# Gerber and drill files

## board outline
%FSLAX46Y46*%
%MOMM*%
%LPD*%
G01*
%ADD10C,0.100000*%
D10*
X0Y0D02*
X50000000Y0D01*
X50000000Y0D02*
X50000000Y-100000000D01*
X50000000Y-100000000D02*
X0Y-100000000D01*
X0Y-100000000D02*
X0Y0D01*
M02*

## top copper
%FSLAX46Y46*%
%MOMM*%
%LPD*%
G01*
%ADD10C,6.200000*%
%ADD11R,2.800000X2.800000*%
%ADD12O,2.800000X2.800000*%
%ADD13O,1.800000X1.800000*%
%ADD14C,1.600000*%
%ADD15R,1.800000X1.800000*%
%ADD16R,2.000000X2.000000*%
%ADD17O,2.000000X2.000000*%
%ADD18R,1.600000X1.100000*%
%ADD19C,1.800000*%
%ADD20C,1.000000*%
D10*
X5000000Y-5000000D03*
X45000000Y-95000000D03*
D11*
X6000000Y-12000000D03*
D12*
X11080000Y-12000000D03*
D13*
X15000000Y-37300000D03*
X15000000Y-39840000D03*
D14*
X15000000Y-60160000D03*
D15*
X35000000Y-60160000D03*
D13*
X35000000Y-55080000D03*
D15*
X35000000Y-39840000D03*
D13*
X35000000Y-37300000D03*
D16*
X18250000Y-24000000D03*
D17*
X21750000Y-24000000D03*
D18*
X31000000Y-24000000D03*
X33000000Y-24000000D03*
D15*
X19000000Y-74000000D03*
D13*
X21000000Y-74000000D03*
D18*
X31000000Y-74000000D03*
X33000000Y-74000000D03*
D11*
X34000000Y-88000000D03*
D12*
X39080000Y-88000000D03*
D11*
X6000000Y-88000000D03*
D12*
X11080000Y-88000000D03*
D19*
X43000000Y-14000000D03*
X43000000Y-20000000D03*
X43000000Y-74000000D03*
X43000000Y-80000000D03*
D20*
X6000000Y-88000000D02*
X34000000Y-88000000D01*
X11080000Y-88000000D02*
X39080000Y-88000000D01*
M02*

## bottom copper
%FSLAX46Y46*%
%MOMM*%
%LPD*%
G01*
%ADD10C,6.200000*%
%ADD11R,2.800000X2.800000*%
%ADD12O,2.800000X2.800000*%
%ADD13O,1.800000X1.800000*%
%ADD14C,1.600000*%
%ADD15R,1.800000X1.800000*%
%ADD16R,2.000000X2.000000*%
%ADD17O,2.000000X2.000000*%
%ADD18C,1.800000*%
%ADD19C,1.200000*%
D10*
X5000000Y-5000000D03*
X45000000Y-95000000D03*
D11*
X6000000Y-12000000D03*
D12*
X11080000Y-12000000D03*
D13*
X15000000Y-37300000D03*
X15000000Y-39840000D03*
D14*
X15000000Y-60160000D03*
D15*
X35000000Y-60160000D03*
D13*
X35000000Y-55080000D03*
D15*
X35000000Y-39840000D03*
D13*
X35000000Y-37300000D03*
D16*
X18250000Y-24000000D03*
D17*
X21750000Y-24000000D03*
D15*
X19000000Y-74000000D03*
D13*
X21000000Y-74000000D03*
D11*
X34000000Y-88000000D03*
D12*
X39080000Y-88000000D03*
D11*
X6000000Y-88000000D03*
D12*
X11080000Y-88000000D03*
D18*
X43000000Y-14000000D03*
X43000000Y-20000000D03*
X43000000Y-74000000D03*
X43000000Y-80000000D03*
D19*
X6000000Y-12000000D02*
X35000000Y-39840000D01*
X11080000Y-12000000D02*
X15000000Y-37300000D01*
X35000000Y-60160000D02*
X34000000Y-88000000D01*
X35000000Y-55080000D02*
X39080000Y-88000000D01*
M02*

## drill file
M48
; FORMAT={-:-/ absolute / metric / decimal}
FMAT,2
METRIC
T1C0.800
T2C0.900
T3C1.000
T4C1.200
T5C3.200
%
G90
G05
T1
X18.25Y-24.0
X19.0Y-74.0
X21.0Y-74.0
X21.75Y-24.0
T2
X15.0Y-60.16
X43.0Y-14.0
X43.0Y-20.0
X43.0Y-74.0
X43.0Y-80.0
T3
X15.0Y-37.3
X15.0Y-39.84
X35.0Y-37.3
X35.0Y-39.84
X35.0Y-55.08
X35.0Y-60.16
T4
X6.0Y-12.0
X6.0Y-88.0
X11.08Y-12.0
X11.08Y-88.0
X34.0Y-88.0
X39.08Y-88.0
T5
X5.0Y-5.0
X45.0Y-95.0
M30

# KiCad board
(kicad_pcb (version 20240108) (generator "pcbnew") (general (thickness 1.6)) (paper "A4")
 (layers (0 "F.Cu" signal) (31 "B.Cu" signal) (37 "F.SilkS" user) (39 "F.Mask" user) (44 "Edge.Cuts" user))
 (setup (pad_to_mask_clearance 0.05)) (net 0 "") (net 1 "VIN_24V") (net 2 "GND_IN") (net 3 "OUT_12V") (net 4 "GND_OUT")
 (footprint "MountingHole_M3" (layer "F.Cu") (at 5 5)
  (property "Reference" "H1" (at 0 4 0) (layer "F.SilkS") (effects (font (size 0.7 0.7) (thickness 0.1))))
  (pad "1" np_thru_hole circle (at 0 0) (size 6.2 6.2) (drill 3.2) (layers "F.Cu" "B.Cu" "F.Mask" "B.Mask")))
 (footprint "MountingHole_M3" (layer "F.Cu") (at 45 95)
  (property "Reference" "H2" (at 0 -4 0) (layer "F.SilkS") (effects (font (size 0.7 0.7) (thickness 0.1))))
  (pad "1" np_thru_hole circle (at 0 0) (size 6.2 6.2) (drill 3.2) (layers "F.Cu" "B.Cu" "F.Mask" "B.Mask")))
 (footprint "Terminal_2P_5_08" (layer "F.Cu") (at 6 12)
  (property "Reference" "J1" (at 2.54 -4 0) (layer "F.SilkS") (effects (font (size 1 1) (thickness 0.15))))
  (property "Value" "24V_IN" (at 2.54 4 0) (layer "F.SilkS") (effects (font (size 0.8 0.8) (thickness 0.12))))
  (pad "1" thru_hole rect (at 0 0) (size 2.8 2.8) (drill 1.2) (layers "F.Cu" "B.Cu" "F.Mask" "B.Mask") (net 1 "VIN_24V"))
  (pad "2" thru_hole oval (at 5.08 0) (size 2.8 2.8) (drill 1.2) (layers "F.Cu" "B.Cu" "F.Mask" "B.Mask") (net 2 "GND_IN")))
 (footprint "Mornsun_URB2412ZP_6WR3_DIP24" (layer "F.Cu") (at 25 50)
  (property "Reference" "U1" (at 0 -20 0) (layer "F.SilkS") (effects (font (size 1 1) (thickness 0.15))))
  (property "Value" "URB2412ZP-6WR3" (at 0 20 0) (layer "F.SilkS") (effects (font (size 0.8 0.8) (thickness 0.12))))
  (pad "2" thru_hole oval (at -10 -12.70) (size 1.8 1.8) (drill 1.0) (layers "F.Cu" "B.Cu" "F.Mask" "B.Mask") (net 2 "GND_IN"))
  (pad "3" thru_hole oval (at -10 -10.16) (size 1.8 1.8) (drill 1.0) (layers "F.Cu" "B.Cu" "F.Mask" "B.Mask") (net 2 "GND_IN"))
  (pad "11" thru_hole circle (at -10 10.16) (size 1.6 1.6) (drill 0.9) (layers "F.Cu" "B.Cu" "F.Mask" "B.Mask"))
  (pad "14" thru_hole rect (at 10 10.16) (size 1.8 1.8) (drill 1.0) (layers "F.Cu" "B.Cu" "F.Mask" "B.Mask") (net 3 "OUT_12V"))
  (pad "16" thru_hole oval (at 10 5.08) (size 1.8 1.8) (drill 1.0) (layers "F.Cu" "B.Cu" "F.Mask" "B.Mask") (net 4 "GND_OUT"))
  (pad "22" thru_hole rect (at 10 -10.16) (size 1.8 1.8) (drill 1.0) (layers "F.Cu" "B.Cu" "F.Mask" "B.Mask") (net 1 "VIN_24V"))
  (pad "23" thru_hole oval (at 10 -12.70) (size 1.8 1.8) (drill 1.0) (layers "F.Cu" "B.Cu" "F.Mask" "B.Mask") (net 1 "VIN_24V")))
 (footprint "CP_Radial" (layer "F.Cu") (at 20 24)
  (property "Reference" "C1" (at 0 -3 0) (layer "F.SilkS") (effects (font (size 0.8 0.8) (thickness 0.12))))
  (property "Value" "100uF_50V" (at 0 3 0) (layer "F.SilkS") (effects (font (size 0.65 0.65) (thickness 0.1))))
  (pad "1" thru_hole rect (at -1.75 0) (size 2 2) (drill 0.8) (layers "F.Cu" "B.Cu" "F.Mask" "B.Mask") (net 1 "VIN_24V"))
  (pad "2" thru_hole oval (at 1.75 0) (size 2 2) (drill 0.8) (layers "F.Cu" "B.Cu" "F.Mask" "B.Mask") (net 2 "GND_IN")))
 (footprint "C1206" (layer "F.Cu") (at 32 24)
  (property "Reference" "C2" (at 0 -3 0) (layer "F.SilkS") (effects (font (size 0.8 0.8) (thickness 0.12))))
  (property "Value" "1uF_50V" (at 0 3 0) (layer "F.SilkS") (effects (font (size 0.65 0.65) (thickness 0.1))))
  (pad "1" smd rect (at -1 0) (size 1.6 1.1) (layers "F.Cu" "F.Mask") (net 1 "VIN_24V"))
  (pad "2" smd rect (at 1 0) (size 1.6 1.1) (layers "F.Cu" "F.Mask") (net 2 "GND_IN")))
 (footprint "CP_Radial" (layer "F.Cu") (at 20 74)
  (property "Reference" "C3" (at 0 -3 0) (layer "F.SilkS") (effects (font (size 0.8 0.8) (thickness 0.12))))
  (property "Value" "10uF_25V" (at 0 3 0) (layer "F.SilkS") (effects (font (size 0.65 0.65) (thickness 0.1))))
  (pad "1" thru_hole rect (at -1 0) (size 1.8 1.8) (drill 0.8) (layers "F.Cu" "B.Cu" "F.Mask" "B.Mask") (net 3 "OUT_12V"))
  (pad "2" thru_hole oval (at 1 0) (size 1.8 1.8) (drill 0.8) (layers "F.Cu" "B.Cu" "F.Mask" "B.Mask") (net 4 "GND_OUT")))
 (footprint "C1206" (layer "F.Cu") (at 32 74)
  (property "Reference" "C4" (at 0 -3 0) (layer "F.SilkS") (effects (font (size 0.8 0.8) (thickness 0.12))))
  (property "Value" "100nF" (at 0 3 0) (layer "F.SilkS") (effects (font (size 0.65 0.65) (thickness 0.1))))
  (pad "1" smd rect (at -1 0) (size 1.6 1.1) (layers "F.Cu" "F.Mask") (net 3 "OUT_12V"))
  (pad "2" smd rect (at 1 0) (size 1.6 1.1) (layers "F.Cu" "F.Mask") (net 4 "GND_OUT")))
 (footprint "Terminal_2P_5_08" (layer "F.Cu") (at 34 88)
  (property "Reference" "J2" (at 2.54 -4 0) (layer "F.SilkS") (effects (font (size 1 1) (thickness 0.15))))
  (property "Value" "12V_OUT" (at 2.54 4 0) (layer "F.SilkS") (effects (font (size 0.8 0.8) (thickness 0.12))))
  (pad "1" thru_hole rect (at 0 0) (size 2.8 2.8) (drill 1.2) (layers "F.Cu" "B.Cu" "F.Mask" "B.Mask") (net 3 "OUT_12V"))
  (pad "2" thru_hole oval (at 5.08 0) (size 2.8 2.8) (drill 1.2) (layers "F.Cu" "B.Cu" "F.Mask" "B.Mask") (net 4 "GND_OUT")))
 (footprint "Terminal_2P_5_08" (layer "F.Cu") (at 6 88)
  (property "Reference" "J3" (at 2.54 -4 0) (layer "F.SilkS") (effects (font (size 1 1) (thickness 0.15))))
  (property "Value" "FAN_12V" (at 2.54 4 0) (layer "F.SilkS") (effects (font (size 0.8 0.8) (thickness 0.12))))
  (pad "1" thru_hole rect (at 0 0) (size 2.8 2.8) (drill 1.2) (layers "F.Cu" "B.Cu" "F.Mask" "B.Mask") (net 3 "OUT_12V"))
  (pad "2" thru_hole oval (at 5.08 0) (size 2.8 2.8) (drill 1.2) (layers "F.Cu" "B.Cu" "F.Mask" "B.Mask") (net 4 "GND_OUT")))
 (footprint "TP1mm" (layer "F.Cu") (at 43 14)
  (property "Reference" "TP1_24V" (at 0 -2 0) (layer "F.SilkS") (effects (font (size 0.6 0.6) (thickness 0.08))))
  (pad "1" thru_hole circle (at 0 0) (size 1.8 1.8) (drill 0.9) (layers "F.Cu" "B.Cu" "F.Mask" "B.Mask") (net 1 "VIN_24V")))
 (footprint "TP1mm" (layer "F.Cu") (at 43 20)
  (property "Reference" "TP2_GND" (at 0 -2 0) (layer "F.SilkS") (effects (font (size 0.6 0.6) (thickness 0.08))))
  (pad "1" thru_hole circle (at 0 0) (size 1.8 1.8) (drill 0.9) (layers "F.Cu" "B.Cu" "F.Mask" "B.Mask") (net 2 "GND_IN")))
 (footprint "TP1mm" (layer "F.Cu") (at 43 74)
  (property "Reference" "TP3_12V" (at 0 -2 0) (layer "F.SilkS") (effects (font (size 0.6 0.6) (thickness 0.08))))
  (pad "1" thru_hole circle (at 0 0) (size 1.8 1.8) (drill 0.9) (layers "F.Cu" "B.Cu" "F.Mask" "B.Mask") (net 3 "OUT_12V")))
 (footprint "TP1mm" (layer "F.Cu") (at 43 80)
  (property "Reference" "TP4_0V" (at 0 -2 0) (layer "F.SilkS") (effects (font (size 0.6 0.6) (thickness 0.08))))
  (pad "1" thru_hole circle (at 0 0) (size 1.8 1.8) (drill 0.9) (layers "F.Cu" "B.Cu" "F.Mask" "B.Mask") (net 4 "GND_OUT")))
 (segment (start 6 12) (end 35 39.84) (width 1.2) (layer "B.Cu") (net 1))
 (segment (start 11.08 12) (end 15 37.3) (width 1.2) (layer "B.Cu") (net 2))
 (segment (start 35 60.16) (end 34 88) (width 1.2) (layer "B.Cu") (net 3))
 (segment (start 35 55.08) (end 39.08 88) (width 1.2) (layer "B.Cu") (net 4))
 (segment (start 6 88) (end 34 88) (width 1.0) (layer "F.Cu") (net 3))
 (segment (start 11.08 88) (end 39.08 88) (width 1.0) (layer "F.Cu") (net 4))
 (gr_line (start 0 0) (end 50 0) (stroke (width 0.1) (type default)) (layer "Edge.Cuts"))
 (gr_line (start 50 0) (end 50 100) (stroke (width 0.1) (type default)) (layer "Edge.Cuts"))
 (gr_line (start 50 100) (end 0 100) (stroke (width 0.1) (type default)) (layer "Edge.Cuts"))
 (gr_line (start 0 100) (end 0 0) (stroke (width 0.1) (type default)) (layer "Edge.Cuts")))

